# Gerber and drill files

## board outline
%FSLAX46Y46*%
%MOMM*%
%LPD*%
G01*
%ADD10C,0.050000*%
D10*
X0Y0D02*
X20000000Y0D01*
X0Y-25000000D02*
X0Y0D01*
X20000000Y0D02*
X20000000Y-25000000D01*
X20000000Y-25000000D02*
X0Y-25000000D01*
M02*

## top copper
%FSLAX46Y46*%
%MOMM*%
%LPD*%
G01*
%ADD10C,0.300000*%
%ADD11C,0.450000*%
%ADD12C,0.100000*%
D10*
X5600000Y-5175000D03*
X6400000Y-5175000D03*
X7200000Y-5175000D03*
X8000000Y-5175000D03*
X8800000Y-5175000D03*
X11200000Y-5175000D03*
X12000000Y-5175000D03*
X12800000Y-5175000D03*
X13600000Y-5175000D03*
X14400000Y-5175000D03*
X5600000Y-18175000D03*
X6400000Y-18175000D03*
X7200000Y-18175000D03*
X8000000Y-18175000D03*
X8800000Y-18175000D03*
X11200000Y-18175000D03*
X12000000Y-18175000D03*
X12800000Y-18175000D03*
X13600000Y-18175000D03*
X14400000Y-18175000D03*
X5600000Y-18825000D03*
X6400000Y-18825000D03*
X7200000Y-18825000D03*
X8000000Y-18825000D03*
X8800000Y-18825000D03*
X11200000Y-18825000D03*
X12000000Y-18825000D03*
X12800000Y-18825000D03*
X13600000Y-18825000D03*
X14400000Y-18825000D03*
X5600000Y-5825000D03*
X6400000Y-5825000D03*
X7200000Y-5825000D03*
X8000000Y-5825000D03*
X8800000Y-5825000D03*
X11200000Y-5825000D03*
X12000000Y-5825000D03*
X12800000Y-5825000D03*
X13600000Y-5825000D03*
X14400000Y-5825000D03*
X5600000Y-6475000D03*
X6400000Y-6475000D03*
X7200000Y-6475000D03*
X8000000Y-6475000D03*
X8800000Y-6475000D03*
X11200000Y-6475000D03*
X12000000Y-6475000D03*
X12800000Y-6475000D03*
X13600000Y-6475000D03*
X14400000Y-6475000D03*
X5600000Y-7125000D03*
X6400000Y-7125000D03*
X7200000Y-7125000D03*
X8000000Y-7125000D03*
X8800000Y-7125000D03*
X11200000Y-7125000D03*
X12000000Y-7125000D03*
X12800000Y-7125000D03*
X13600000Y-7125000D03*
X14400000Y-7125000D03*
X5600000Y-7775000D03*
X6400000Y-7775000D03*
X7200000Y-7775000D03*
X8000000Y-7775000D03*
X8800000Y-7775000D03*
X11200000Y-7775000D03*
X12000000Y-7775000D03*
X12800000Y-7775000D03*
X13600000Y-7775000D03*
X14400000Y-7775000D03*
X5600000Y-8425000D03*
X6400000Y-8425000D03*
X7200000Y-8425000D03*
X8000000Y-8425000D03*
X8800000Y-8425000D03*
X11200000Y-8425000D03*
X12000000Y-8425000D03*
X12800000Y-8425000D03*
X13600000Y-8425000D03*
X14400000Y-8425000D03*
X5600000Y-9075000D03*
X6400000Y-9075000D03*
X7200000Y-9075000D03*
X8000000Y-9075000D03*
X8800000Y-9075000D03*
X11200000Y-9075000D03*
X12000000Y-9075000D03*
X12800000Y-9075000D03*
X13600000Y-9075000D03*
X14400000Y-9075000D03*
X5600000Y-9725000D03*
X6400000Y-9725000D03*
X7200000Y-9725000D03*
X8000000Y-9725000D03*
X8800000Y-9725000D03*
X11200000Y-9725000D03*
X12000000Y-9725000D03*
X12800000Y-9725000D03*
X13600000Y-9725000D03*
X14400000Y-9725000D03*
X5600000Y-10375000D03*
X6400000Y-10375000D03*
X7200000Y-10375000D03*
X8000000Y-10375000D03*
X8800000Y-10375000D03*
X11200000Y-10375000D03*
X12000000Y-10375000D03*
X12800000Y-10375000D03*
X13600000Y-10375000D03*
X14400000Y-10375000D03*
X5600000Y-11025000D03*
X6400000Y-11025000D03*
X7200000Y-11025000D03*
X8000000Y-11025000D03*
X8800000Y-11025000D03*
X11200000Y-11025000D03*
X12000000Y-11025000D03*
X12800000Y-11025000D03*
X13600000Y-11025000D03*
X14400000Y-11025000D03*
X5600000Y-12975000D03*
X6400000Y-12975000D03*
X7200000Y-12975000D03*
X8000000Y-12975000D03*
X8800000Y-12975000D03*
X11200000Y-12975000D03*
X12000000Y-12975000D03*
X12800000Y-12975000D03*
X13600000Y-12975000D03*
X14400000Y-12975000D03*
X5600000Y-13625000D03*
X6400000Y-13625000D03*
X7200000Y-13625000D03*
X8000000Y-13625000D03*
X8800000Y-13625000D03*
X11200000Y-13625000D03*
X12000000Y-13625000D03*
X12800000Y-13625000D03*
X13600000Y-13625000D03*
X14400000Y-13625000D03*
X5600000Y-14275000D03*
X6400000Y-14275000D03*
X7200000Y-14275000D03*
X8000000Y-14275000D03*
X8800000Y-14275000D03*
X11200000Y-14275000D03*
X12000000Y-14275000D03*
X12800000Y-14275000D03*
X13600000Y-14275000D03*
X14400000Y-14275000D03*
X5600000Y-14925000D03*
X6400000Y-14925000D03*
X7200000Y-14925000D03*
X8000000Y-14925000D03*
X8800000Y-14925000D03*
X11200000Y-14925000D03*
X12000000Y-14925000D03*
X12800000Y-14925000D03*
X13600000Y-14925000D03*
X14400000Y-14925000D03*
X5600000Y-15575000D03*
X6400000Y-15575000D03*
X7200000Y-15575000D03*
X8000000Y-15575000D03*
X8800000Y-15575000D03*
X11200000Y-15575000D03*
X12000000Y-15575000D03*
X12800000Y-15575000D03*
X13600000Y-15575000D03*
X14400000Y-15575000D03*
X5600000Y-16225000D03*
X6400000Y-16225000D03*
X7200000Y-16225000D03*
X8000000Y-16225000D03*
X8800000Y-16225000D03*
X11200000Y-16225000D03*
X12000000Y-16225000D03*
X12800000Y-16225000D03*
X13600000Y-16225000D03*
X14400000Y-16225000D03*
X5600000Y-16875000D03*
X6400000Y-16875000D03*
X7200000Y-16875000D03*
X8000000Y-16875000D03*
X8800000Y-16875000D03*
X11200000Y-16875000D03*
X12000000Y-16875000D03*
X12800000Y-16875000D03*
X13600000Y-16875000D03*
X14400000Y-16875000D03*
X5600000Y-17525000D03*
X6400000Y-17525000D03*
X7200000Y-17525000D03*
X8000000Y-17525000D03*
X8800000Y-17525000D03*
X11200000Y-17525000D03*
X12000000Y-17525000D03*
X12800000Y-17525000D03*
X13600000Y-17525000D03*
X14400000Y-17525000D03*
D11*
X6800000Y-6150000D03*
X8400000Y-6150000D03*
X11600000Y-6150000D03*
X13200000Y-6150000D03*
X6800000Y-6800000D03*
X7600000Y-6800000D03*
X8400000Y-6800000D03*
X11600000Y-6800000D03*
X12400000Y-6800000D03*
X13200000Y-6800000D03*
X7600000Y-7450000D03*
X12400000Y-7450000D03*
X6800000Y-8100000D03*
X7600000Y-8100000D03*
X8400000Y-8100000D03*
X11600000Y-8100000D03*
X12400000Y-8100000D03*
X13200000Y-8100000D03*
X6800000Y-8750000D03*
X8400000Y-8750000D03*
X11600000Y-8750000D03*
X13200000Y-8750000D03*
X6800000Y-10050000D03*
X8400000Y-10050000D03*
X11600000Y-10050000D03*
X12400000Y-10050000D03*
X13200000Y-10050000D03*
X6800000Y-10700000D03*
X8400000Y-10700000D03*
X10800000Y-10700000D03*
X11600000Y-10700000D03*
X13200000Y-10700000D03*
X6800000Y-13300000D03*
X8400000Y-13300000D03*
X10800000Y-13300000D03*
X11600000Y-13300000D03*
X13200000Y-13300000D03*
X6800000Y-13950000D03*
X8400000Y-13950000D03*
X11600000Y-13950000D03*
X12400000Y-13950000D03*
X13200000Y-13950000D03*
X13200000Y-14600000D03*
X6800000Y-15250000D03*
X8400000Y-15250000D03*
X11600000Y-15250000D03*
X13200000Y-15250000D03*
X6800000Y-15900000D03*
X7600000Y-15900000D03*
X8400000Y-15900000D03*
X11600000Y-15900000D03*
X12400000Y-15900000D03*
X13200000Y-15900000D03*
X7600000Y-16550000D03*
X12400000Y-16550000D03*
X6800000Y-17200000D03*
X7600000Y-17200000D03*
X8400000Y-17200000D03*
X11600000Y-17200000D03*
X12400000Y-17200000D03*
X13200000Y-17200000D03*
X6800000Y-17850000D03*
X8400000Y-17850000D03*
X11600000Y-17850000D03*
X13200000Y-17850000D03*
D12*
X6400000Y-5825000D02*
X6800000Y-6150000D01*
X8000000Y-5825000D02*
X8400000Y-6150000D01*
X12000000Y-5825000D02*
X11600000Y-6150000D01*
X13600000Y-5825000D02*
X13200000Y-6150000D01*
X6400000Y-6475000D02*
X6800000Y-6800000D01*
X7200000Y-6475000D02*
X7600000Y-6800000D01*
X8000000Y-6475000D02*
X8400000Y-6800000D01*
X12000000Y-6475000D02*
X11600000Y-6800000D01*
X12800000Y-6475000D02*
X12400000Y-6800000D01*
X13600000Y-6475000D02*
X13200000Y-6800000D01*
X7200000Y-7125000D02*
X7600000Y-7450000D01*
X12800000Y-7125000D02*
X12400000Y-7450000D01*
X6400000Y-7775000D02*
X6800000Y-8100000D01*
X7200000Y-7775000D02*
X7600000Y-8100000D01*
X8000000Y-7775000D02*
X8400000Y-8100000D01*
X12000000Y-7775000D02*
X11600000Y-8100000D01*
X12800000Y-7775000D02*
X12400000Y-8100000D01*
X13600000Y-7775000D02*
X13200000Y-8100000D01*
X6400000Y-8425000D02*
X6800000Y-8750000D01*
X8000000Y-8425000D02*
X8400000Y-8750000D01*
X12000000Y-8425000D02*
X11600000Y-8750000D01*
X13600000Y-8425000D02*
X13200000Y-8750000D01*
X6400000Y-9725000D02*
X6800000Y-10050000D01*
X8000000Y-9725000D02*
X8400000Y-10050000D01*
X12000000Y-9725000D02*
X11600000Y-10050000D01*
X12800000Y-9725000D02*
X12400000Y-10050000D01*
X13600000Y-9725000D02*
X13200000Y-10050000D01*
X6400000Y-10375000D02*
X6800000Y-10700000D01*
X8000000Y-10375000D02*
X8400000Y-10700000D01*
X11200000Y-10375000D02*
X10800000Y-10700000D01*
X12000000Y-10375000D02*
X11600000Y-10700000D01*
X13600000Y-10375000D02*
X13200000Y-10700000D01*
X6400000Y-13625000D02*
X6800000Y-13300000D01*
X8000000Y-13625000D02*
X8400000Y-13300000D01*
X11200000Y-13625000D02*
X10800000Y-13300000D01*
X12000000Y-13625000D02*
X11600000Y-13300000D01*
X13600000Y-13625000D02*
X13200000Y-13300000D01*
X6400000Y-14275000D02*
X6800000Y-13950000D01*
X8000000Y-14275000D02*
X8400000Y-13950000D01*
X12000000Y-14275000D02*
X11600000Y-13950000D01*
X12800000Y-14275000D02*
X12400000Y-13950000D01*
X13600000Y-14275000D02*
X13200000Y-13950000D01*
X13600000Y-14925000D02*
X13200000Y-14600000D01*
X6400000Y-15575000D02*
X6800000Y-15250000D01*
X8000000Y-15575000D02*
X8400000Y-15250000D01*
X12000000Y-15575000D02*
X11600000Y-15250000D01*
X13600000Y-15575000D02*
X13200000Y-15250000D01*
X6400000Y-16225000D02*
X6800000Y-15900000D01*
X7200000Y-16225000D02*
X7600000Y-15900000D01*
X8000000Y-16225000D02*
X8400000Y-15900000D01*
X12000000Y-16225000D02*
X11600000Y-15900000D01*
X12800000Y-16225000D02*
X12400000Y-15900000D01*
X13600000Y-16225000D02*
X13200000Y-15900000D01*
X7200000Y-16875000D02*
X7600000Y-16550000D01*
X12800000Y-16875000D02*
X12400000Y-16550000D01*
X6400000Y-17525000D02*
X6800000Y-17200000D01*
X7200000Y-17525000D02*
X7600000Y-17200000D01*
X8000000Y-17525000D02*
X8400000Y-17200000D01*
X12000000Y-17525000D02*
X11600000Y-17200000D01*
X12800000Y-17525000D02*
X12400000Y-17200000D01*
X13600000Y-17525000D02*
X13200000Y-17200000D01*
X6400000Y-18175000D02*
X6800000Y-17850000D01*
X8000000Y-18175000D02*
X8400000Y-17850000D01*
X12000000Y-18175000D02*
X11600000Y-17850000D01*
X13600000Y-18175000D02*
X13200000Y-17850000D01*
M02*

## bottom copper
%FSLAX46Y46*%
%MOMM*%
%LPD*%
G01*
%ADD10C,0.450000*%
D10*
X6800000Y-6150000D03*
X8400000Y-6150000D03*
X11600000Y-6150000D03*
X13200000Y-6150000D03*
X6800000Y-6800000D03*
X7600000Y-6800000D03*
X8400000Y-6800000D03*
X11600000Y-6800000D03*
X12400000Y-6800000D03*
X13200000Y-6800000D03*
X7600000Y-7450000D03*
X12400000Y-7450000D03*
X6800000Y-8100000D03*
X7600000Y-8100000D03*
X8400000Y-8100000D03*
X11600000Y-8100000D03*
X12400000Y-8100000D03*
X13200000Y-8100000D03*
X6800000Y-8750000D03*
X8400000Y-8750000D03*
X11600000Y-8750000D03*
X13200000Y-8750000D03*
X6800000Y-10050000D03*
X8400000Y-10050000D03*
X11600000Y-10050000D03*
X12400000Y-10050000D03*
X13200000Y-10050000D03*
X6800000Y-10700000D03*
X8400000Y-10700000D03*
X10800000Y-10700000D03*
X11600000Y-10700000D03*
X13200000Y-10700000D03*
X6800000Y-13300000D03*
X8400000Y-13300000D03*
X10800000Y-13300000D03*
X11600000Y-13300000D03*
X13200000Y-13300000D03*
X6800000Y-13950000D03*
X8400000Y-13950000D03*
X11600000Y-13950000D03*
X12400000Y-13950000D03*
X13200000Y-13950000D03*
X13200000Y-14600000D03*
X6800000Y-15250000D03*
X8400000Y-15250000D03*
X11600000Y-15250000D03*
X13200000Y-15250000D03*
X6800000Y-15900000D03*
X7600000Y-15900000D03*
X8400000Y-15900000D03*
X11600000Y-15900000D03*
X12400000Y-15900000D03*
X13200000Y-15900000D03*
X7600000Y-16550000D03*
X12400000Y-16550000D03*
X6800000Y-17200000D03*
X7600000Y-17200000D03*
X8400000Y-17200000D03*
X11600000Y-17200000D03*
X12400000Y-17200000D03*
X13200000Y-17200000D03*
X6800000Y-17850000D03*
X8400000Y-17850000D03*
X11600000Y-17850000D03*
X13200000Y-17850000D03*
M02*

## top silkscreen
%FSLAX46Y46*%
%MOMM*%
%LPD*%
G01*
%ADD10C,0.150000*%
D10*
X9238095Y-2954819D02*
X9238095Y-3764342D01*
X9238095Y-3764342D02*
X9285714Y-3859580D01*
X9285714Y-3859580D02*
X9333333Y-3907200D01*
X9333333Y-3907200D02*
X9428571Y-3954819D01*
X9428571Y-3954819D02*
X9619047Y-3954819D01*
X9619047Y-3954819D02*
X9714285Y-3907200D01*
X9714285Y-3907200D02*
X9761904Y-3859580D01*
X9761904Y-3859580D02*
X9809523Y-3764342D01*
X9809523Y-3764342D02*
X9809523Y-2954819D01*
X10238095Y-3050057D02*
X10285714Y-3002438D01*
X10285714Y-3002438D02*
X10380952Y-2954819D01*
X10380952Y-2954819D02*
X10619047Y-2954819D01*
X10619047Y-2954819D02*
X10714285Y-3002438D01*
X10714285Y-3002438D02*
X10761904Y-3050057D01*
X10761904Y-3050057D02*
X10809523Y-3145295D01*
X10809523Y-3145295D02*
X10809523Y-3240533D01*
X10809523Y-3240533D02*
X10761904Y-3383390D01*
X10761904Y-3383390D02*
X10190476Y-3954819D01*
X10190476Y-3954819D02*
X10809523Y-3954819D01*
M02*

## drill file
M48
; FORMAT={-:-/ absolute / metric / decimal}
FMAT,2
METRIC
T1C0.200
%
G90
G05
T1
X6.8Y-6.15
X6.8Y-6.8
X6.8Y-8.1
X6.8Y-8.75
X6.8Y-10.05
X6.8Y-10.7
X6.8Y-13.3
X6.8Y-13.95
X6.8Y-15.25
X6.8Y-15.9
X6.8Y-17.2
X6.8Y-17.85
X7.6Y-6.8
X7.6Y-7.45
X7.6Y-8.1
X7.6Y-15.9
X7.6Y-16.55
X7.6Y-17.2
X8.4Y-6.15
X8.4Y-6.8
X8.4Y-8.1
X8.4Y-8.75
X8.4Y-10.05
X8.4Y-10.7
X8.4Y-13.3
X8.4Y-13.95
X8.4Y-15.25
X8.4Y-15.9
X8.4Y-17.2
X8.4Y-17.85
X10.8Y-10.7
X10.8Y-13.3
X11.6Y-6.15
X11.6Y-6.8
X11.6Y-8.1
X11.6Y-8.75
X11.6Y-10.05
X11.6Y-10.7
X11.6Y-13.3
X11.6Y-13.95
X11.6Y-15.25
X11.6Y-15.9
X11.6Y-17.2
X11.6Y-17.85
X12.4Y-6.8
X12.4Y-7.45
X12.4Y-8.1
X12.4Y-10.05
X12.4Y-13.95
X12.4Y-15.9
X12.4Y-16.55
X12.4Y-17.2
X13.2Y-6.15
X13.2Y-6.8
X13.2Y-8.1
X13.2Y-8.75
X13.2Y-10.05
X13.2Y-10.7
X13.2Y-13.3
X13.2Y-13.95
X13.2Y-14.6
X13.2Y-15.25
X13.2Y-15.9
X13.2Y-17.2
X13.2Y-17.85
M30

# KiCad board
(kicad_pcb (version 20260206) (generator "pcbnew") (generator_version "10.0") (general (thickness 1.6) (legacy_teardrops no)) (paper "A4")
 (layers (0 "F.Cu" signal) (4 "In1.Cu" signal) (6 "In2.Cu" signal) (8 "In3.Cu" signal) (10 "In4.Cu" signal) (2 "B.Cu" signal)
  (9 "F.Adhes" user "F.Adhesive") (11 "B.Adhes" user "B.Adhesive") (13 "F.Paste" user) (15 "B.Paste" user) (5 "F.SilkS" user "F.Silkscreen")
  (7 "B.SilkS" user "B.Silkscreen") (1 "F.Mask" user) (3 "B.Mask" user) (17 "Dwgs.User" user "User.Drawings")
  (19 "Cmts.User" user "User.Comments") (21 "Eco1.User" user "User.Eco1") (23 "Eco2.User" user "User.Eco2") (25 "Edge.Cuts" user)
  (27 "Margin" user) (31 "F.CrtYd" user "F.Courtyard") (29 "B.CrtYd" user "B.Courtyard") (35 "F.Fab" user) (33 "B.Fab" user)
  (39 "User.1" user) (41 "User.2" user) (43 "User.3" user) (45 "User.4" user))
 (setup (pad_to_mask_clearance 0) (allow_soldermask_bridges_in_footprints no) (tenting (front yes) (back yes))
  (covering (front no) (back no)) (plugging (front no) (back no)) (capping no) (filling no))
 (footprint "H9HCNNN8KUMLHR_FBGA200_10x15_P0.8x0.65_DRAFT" (layer "F.Cu") (at 10 12)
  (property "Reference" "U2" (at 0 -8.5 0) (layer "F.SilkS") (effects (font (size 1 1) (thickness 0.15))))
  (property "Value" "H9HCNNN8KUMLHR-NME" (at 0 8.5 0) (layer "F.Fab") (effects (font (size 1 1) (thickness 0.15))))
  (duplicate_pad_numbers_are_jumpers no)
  (pad "A1" smd circle (at -4.4 -6.825) (size 0.3 0.3) (layers "F.Cu" "F.Mask" "F.Paste"))
  (pad "A2" smd circle (at -3.6 -6.825) (size 0.3 0.3) (layers "F.Cu" "F.Mask" "F.Paste"))
  (pad "A3" smd circle (at -2.8 -6.825) (size 0.3 0.3) (layers "F.Cu" "F.Mask" "F.Paste") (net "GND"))
  (pad "A4" smd circle (at -2 -6.825) (size 0.3 0.3) (layers "F.Cu" "F.Mask" "F.Paste") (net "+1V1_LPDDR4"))
  (pad "A5" smd circle (at -1.2 -6.825) (size 0.3 0.3) (layers "F.Cu" "F.Mask" "F.Paste") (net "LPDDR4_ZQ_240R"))
  (pad "A8" smd circle (at 1.2 -6.825) (size 0.3 0.3) (layers "F.Cu" "F.Mask" "F.Paste"))
  (pad "A9" smd circle (at 2 -6.825) (size 0.3 0.3) (layers "F.Cu" "F.Mask" "F.Paste") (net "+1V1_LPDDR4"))
  (pad "A10" smd circle (at 2.8 -6.825) (size 0.3 0.3) (layers "F.Cu" "F.Mask" "F.Paste") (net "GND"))
  (pad "A11" smd circle (at 3.6 -6.825) (size 0.3 0.3) (layers "F.Cu" "F.Mask" "F.Paste"))
  (pad "A12" smd circle (at 4.4 -6.825) (size 0.3 0.3) (layers "F.Cu" "F.Mask" "F.Paste"))
  (pad "AA1" smd circle (at -4.4 6.175) (size 0.3 0.3) (layers "F.Cu" "F.Mask" "F.Paste"))
  (pad "AA2" smd circle (at -3.6 6.175) (size 0.3 0.3) (layers "F.Cu" "F.Mask" "F.Paste") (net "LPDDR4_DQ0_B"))
  (pad "AA3" smd circle (at -2.8 6.175) (size 0.3 0.3) (layers "F.Cu" "F.Mask" "F.Paste") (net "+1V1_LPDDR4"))
  (pad "AA4" smd circle (at -2 6.175) (size 0.3 0.3) (layers "F.Cu" "F.Mask" "F.Paste") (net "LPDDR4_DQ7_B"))
  (pad "AA5" smd circle (at -1.2 6.175) (size 0.3 0.3) (layers "F.Cu" "F.Mask" "F.Paste") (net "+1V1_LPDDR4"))
  (pad "AA8" smd circle (at 1.2 6.175) (size 0.3 0.3) (layers "F.Cu" "F.Mask" "F.Paste") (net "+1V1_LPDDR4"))
  (pad "AA9" smd circle (at 2 6.175) (size 0.3 0.3) (layers "F.Cu" "F.Mask" "F.Paste") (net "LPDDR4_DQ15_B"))
  (pad "AA10" smd circle (at 2.8 6.175) (size 0.3 0.3) (layers "F.Cu" "F.Mask" "F.Paste") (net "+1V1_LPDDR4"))
  (pad "AA11" smd circle (at 3.6 6.175) (size 0.3 0.3) (layers "F.Cu" "F.Mask" "F.Paste") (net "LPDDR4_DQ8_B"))
  (pad "AA12" smd circle (at 4.4 6.175) (size 0.3 0.3) (layers "F.Cu" "F.Mask" "F.Paste"))
  (pad "AB1" smd circle (at -4.4 6.825) (size 0.3 0.3) (layers "F.Cu" "F.Mask" "F.Paste"))
  (pad "AB2" smd circle (at -3.6 6.825) (size 0.3 0.3) (layers "F.Cu" "F.Mask" "F.Paste"))
  (pad "AB3" smd circle (at -2.8 6.825) (size 0.3 0.3) (layers "F.Cu" "F.Mask" "F.Paste") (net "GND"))
  (pad "AB4" smd circle (at -2 6.825) (size 0.3 0.3) (layers "F.Cu" "F.Mask" "F.Paste") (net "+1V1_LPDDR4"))
  (pad "AB5" smd circle (at -1.2 6.825) (size 0.3 0.3) (layers "F.Cu" "F.Mask" "F.Paste") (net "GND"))
  (pad "AB8" smd circle (at 1.2 6.825) (size 0.3 0.3) (layers "F.Cu" "F.Mask" "F.Paste") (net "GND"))
  (pad "AB9" smd circle (at 2 6.825) (size 0.3 0.3) (layers "F.Cu" "F.Mask" "F.Paste") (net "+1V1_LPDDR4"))
  (pad "AB10" smd circle (at 2.8 6.825) (size 0.3 0.3) (layers "F.Cu" "F.Mask" "F.Paste") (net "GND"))
  (pad "AB11" smd circle (at 3.6 6.825) (size 0.3 0.3) (layers "F.Cu" "F.Mask" "F.Paste"))
  (pad "AB12" smd circle (at 4.4 6.825) (size 0.3 0.3) (layers "F.Cu" "F.Mask" "F.Paste"))
  (pad "B1" smd circle (at -4.4 -6.175) (size 0.3 0.3) (layers "F.Cu" "F.Mask" "F.Paste"))
  (pad "B2" smd circle (at -3.6 -6.175) (size 0.3 0.3) (layers "F.Cu" "F.Mask" "F.Paste") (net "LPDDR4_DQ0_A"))
  (pad "B3" smd circle (at -2.8 -6.175) (size 0.3 0.3) (layers "F.Cu" "F.Mask" "F.Paste") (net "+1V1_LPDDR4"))
  (pad "B4" smd circle (at -2 -6.175) (size 0.3 0.3) (layers "F.Cu" "F.Mask" "F.Paste") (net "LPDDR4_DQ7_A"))
  (pad "B5" smd circle (at -1.2 -6.175) (size 0.3 0.3) (layers "F.Cu" "F.Mask" "F.Paste") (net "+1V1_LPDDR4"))
  (pad "B8" smd circle (at 1.2 -6.175) (size 0.3 0.3) (layers "F.Cu" "F.Mask" "F.Paste") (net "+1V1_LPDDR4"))
  (pad "B9" smd circle (at 2 -6.175) (size 0.3 0.3) (layers "F.Cu" "F.Mask" "F.Paste") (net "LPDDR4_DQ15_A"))
  (pad "B10" smd circle (at 2.8 -6.175) (size 0.3 0.3) (layers "F.Cu" "F.Mask" "F.Paste") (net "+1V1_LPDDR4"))
  (pad "B11" smd circle (at 3.6 -6.175) (size 0.3 0.3) (layers "F.Cu" "F.Mask" "F.Paste") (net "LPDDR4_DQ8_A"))
  (pad "B12" smd circle (at 4.4 -6.175) (size 0.3 0.3) (layers "F.Cu" "F.Mask" "F.Paste"))
  (pad "C1" smd circle (at -4.4 -5.525) (size 0.3 0.3) (layers "F.Cu" "F.Mask" "F.Paste") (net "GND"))
  (pad "C2" smd circle (at -3.6 -5.525) (size 0.3 0.3) (layers "F.Cu" "F.Mask" "F.Paste") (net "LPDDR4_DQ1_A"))
  (pad "C3" smd circle (at -2.8 -5.525) (size 0.3 0.3) (layers "F.Cu" "F.Mask" "F.Paste") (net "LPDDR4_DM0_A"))
  (pad "C4" smd circle (at -2 -5.525) (size 0.3 0.3) (layers "F.Cu" "F.Mask" "F.Paste") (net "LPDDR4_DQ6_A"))
  (pad "C5" smd circle (at -1.2 -5.525) (size 0.3 0.3) (layers "F.Cu" "F.Mask" "F.Paste") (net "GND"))
  (pad "C8" smd circle (at 1.2 -5.525) (size 0.3 0.3) (layers "F.Cu" "F.Mask" "F.Paste") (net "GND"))
  (pad "C9" smd circle (at 2 -5.525) (size 0.3 0.3) (layers "F.Cu" "F.Mask" "F.Paste") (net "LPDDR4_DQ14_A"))
  (pad "C10" smd circle (at 2.8 -5.525) (size 0.3 0.3) (layers "F.Cu" "F.Mask" "F.Paste") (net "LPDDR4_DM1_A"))
  (pad "C11" smd circle (at 3.6 -5.525) (size 0.3 0.3) (layers "F.Cu" "F.Mask" "F.Paste") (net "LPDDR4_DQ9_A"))
  (pad "C12" smd circle (at 4.4 -5.525) (size 0.3 0.3) (layers "F.Cu" "F.Mask" "F.Paste") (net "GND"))
  (pad "D1" smd circle (at -4.4 -4.875) (size 0.3 0.3) (layers "F.Cu" "F.Mask" "F.Paste") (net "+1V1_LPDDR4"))
  (pad "D2" smd circle (at -3.6 -4.875) (size 0.3 0.3) (layers "F.Cu" "F.Mask" "F.Paste") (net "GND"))
  (pad "D3" smd circle (at -2.8 -4.875) (size 0.3 0.3) (layers "F.Cu" "F.Mask" "F.Paste") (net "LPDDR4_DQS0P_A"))
  (pad "D4" smd circle (at -2 -4.875) (size 0.3 0.3) (layers "F.Cu" "F.Mask" "F.Paste") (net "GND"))
  (pad "D5" smd circle (at -1.2 -4.875) (size 0.3 0.3) (layers "F.Cu" "F.Mask" "F.Paste") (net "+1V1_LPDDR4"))
  (pad "D8" smd circle (at 1.2 -4.875) (size 0.3 0.3) (layers "F.Cu" "F.Mask" "F.Paste") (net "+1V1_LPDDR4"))
  (pad "D9" smd circle (at 2 -4.875) (size 0.3 0.3) (layers "F.Cu" "F.Mask" "F.Paste") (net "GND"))
  (pad "D10" smd circle (at 2.8 -4.875) (size 0.3 0.3) (layers "F.Cu" "F.Mask" "F.Paste") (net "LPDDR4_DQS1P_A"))
  (pad "D11" smd circle (at 3.6 -4.875) (size 0.3 0.3) (layers "F.Cu" "F.Mask" "F.Paste") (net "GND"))
  (pad "D12" smd circle (at 4.4 -4.875) (size 0.3 0.3) (layers "F.Cu" "F.Mask" "F.Paste") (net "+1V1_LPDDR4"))
  (pad "E1" smd circle (at -4.4 -4.225) (size 0.3 0.3) (layers "F.Cu" "F.Mask" "F.Paste") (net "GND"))
  (pad "E2" smd circle (at -3.6 -4.225) (size 0.3 0.3) (layers "F.Cu" "F.Mask" "F.Paste") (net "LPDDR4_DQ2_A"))
  (pad "E3" smd circle (at -2.8 -4.225) (size 0.3 0.3) (layers "F.Cu" "F.Mask" "F.Paste") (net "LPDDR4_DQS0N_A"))
  (pad "E4" smd circle (at -2 -4.225) (size 0.3 0.3) (layers "F.Cu" "F.Mask" "F.Paste") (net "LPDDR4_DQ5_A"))
  (pad "E5" smd circle (at -1.2 -4.225) (size 0.3 0.3) (layers "F.Cu" "F.Mask" "F.Paste") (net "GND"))
  (pad "E8" smd circle (at 1.2 -4.225) (size 0.3 0.3) (layers "F.Cu" "F.Mask" "F.Paste") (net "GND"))
  (pad "E9" smd circle (at 2 -4.225) (size 0.3 0.3) (layers "F.Cu" "F.Mask" "F.Paste") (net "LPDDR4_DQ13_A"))
  (pad "E10" smd circle (at 2.8 -4.225) (size 0.3 0.3) (layers "F.Cu" "F.Mask" "F.Paste") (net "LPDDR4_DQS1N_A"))
  (pad "E11" smd circle (at 3.6 -4.225) (size 0.3 0.3) (layers "F.Cu" "F.Mask" "F.Paste") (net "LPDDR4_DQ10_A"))
  (pad "E12" smd circle (at 4.4 -4.225) (size 0.3 0.3) (layers "F.Cu" "F.Mask" "F.Paste") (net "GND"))
  (pad "F1" smd circle (at -4.4 -3.575) (size 0.3 0.3) (layers "F.Cu" "F.Mask" "F.Paste") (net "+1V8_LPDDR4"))
  (pad "F2" smd circle (at -3.6 -3.575) (size 0.3 0.3) (layers "F.Cu" "F.Mask" "F.Paste") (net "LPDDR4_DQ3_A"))
  (pad "F3" smd circle (at -2.8 -3.575) (size 0.3 0.3) (layers "F.Cu" "F.Mask" "F.Paste") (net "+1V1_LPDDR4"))
  (pad "F4" smd circle (at -2 -3.575) (size 0.3 0.3) (layers "F.Cu" "F.Mask" "F.Paste") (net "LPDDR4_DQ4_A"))
  (pad "F5" smd circle (at -1.2 -3.575) (size 0.3 0.3) (layers "F.Cu" "F.Mask" "F.Paste") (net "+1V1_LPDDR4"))
  (pad "F8" smd circle (at 1.2 -3.575) (size 0.3 0.3) (layers "F.Cu" "F.Mask" "F.Paste") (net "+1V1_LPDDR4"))
  (pad "F9" smd circle (at 2 -3.575) (size 0.3 0.3) (layers "F.Cu" "F.Mask" "F.Paste") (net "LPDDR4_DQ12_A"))
  (pad "F10" smd circle (at 2.8 -3.575) (size 0.3 0.3) (layers "F.Cu" "F.Mask" "F.Paste") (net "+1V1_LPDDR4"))
  (pad "F11" smd circle (at 3.6 -3.575) (size 0.3 0.3) (layers "F.Cu" "F.Mask" "F.Paste") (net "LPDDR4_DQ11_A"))
  (pad "F12" smd circle (at 4.4 -3.575) (size 0.3 0.3) (layers "F.Cu" "F.Mask" "F.Paste") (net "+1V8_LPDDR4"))
  (pad "G1" smd circle (at -4.4 -2.925) (size 0.3 0.3) (layers "F.Cu" "F.Mask" "F.Paste") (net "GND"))
  (pad "G2" smd circle (at -3.6 -2.925) (size 0.3 0.3) (layers "F.Cu" "F.Mask" "F.Paste") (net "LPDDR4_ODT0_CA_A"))
  (pad "G3" smd circle (at -2.8 -2.925) (size 0.3 0.3) (layers "F.Cu" "F.Mask" "F.Paste") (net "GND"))
  (pad "G4" smd circle (at -2 -2.925) (size 0.3 0.3) (layers "F.Cu" "F.Mask" "F.Paste") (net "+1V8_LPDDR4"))
  (pad "G5" smd circle (at -1.2 -2.925) (size 0.3 0.3) (layers "F.Cu" "F.Mask" "F.Paste") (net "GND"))
  (pad "G8" smd circle (at 1.2 -2.925) (size 0.3 0.3) (layers "F.Cu" "F.Mask" "F.Paste") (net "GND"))
  (pad "G9" smd circle (at 2 -2.925) (size 0.3 0.3) (layers "F.Cu" "F.Mask" "F.Paste") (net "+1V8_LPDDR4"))
  (pad "G10" smd circle (at 2.8 -2.925) (size 0.3 0.3) (layers "F.Cu" "F.Mask" "F.Paste") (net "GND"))
  (pad "G11" smd circle (at 3.6 -2.925) (size 0.3 0.3) (layers "F.Cu" "F.Mask" "F.Paste"))
  (pad "G12" smd circle (at 4.4 -2.925) (size 0.3 0.3) (layers "F.Cu" "F.Mask" "F.Paste") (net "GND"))
  (pad "H1" smd circle (at -4.4 -2.275) (size 0.3 0.3) (layers "F.Cu" "F.Mask" "F.Paste") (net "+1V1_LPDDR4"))
  (pad "H2" smd circle (at -3.6 -2.275) (size 0.3 0.3) (layers "F.Cu" "F.Mask" "F.Paste") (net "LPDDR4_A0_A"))
  (pad "H3" smd circle (at -2.8 -2.275) (size 0.3 0.3) (layers "F.Cu" "F.Mask" "F.Paste"))
  (pad "H4" smd circle (at -2 -2.275) (size 0.3 0.3) (layers "F.Cu" "F.Mask" "F.Paste") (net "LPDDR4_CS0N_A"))
  (pad "H5" smd circle (at -1.2 -2.275) (size 0.3 0.3) (layers "F.Cu" "F.Mask" "F.Paste") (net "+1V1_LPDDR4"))
  (pad "H8" smd circle (at 1.2 -2.275) (size 0.3 0.3) (layers "F.Cu" "F.Mask" "F.Paste") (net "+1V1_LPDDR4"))
  (pad "H9" smd circle (at 2 -2.275) (size 0.3 0.3) (layers "F.Cu" "F.Mask" "F.Paste") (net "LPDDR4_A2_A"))
  (pad "H10" smd circle (at 2.8 -2.275) (size 0.3 0.3) (layers "F.Cu" "F.Mask" "F.Paste") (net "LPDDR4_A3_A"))
  (pad "H11" smd circle (at 3.6 -2.275) (size 0.3 0.3) (layers "F.Cu" "F.Mask" "F.Paste") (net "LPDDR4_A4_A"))
  (pad "H12" smd circle (at 4.4 -2.275) (size 0.3 0.3) (layers "F.Cu" "F.Mask" "F.Paste") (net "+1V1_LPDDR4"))
  (pad "J1" smd circle (at -4.4 -1.625) (size 0.3 0.3) (layers "F.Cu" "F.Mask" "F.Paste") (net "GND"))
  (pad "J2" smd circle (at -3.6 -1.625) (size 0.3 0.3) (layers "F.Cu" "F.Mask" "F.Paste") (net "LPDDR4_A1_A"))
  (pad "J3" smd circle (at -2.8 -1.625) (size 0.3 0.3) (layers "F.Cu" "F.Mask" "F.Paste") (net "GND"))
  (pad "J4" smd circle (at -2 -1.625) (size 0.3 0.3) (layers "F.Cu" "F.Mask" "F.Paste") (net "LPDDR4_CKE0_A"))
  (pad "J5" smd circle (at -1.2 -1.625) (size 0.3 0.3) (layers "F.Cu" "F.Mask" "F.Paste"))
  (pad "J8" smd circle (at 1.2 -1.625) (size 0.3 0.3) (layers "F.Cu" "F.Mask" "F.Paste") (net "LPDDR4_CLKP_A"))
  (pad "J9" smd circle (at 2 -1.625) (size 0.3 0.3) (layers "F.Cu" "F.Mask" "F.Paste") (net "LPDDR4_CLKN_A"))
  (pad "J10" smd circle (at 2.8 -1.625) (size 0.3 0.3) (layers "F.Cu" "F.Mask" "F.Paste") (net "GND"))
  (pad "J11" smd circle (at 3.6 -1.625) (size 0.3 0.3) (layers "F.Cu" "F.Mask" "F.Paste") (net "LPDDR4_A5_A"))
  (pad "J12" smd circle (at 4.4 -1.625) (size 0.3 0.3) (layers "F.Cu" "F.Mask" "F.Paste") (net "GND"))
  (pad "K1" smd circle (at -4.4 -0.975) (size 0.3 0.3) (layers "F.Cu" "F.Mask" "F.Paste") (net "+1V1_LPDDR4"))
  (pad "K2" smd circle (at -3.6 -0.975) (size 0.3 0.3) (layers "F.Cu" "F.Mask" "F.Paste") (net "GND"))
  (pad "K3" smd circle (at -2.8 -0.975) (size 0.3 0.3) (layers "F.Cu" "F.Mask" "F.Paste") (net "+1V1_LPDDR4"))
  (pad "K4" smd circle (at -2 -0.975) (size 0.3 0.3) (layers "F.Cu" "F.Mask" "F.Paste") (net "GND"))
  (pad "K5" smd circle (at -1.2 -0.975) (size 0.3 0.3) (layers "F.Cu" "F.Mask" "F.Paste"))
  (pad "K8" smd circle (at 1.2 -0.975) (size 0.3 0.3) (layers "F.Cu" "F.Mask" "F.Paste"))
  (pad "K9" smd circle (at 2 -0.975) (size 0.3 0.3) (layers "F.Cu" "F.Mask" "F.Paste") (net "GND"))
  (pad "K10" smd circle (at 2.8 -0.975) (size 0.3 0.3) (layers "F.Cu" "F.Mask" "F.Paste") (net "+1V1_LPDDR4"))
  (pad "K11" smd circle (at 3.6 -0.975) (size 0.3 0.3) (layers "F.Cu" "F.Mask" "F.Paste") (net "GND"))
  (pad "K12" smd circle (at 4.4 -0.975) (size 0.3 0.3) (layers "F.Cu" "F.Mask" "F.Paste") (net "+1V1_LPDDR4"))
  (pad "N1" smd circle (at -4.4 0.975) (size 0.3 0.3) (layers "F.Cu" "F.Mask" "F.Paste") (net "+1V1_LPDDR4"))
  (pad "N2" smd circle (at -3.6 0.975) (size 0.3 0.3) (layers "F.Cu" "F.Mask" "F.Paste") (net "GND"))
  (pad "N3" smd circle (at -2.8 0.975) (size 0.3 0.3) (layers "F.Cu" "F.Mask" "F.Paste") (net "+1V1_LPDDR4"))
  (pad "N4" smd circle (at -2 0.975) (size 0.3 0.3) (layers "F.Cu" "F.Mask" "F.Paste") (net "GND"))
  (pad "N5" smd circle (at -1.2 0.975) (size 0.3 0.3) (layers "F.Cu" "F.Mask" "F.Paste"))
  (pad "N8" smd circle (at 1.2 0.975) (size 0.3 0.3) (layers "F.Cu" "F.Mask" "F.Paste"))
  (pad "N9" smd circle (at 2 0.975) (size 0.3 0.3) (layers "F.Cu" "F.Mask" "F.Paste") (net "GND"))
  (pad "N10" smd circle (at 2.8 0.975) (size 0.3 0.3) (layers "F.Cu" "F.Mask" "F.Paste") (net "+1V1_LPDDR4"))
  (pad "N11" smd circle (at 3.6 0.975) (size 0.3 0.3) (layers "F.Cu" "F.Mask" "F.Paste") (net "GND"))
  (pad "N12" smd circle (at 4.4 0.975) (size 0.3 0.3) (layers "F.Cu" "F.Mask" "F.Paste") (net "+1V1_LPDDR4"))
  (pad "P1" smd circle (at -4.4 1.625) (size 0.3 0.3) (layers "F.Cu" "F.Mask" "F.Paste") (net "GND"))
  (pad "P2" smd circle (at -3.6 1.625) (size 0.3 0.3) (layers "F.Cu" "F.Mask" "F.Paste") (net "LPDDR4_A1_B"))
  (pad "P3" smd circle (at -2.8 1.625) (size 0.3 0.3) (layers "F.Cu" "F.Mask" "F.Paste") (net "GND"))
  (pad "P4" smd circle (at -2 1.625) (size 0.3 0.3) (layers "F.Cu" "F.Mask" "F.Paste") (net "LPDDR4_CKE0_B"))
  (pad "P5" smd circle (at -1.2 1.625) (size 0.3 0.3) (layers "F.Cu" "F.Mask" "F.Paste"))
  (pad "P8" smd circle (at 1.2 1.625) (size 0.3 0.3) (layers "F.Cu" "F.Mask" "F.Paste") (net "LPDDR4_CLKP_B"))
  (pad "P9" smd circle (at 2 1.625) (size 0.3 0.3) (layers "F.Cu" "F.Mask" "F.Paste") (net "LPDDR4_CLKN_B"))
  (pad "P10" smd circle (at 2.8 1.625) (size 0.3 0.3) (layers "F.Cu" "F.Mask" "F.Paste") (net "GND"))
  (pad "P11" smd circle (at 3.6 1.625) (size 0.3 0.3) (layers "F.Cu" "F.Mask" "F.Paste") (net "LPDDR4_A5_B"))
  (pad "P12" smd circle (at 4.4 1.625) (size 0.3 0.3) (layers "F.Cu" "F.Mask" "F.Paste") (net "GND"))
  (pad "R1" smd circle (at -4.4 2.275) (size 0.3 0.3) (layers "F.Cu" "F.Mask" "F.Paste") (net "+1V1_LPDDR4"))
  (pad "R2" smd circle (at -3.6 2.275) (size 0.3 0.3) (layers "F.Cu" "F.Mask" "F.Paste") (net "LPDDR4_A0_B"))
  (pad "R3" smd circle (at -2.8 2.275) (size 0.3 0.3) (layers "F.Cu" "F.Mask" "F.Paste"))
  (pad "R4" smd circle (at -2 2.275) (size 0.3 0.3) (layers "F.Cu" "F.Mask" "F.Paste") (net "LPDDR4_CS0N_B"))
  (pad "R5" smd circle (at -1.2 2.275) (size 0.3 0.3) (layers "F.Cu" "F.Mask" "F.Paste") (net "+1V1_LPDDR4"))
  (pad "R8" smd circle (at 1.2 2.275) (size 0.3 0.3) (layers "F.Cu" "F.Mask" "F.Paste") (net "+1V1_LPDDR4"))
  (pad "R9" smd circle (at 2 2.275) (size 0.3 0.3) (layers "F.Cu" "F.Mask" "F.Paste") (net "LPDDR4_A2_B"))
  (pad "R10" smd circle (at 2.8 2.275) (size 0.3 0.3) (layers "F.Cu" "F.Mask" "F.Paste") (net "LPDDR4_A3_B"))
  (pad "R11" smd circle (at 3.6 2.275) (size 0.3 0.3) (layers "F.Cu" "F.Mask" "F.Paste") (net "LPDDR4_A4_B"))
  (pad "R12" smd circle (at 4.4 2.275) (size 0.3 0.3) (layers "F.Cu" "F.Mask" "F.Paste") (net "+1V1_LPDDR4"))
  (pad "T1" smd circle (at -4.4 2.925) (size 0.3 0.3) (layers "F.Cu" "F.Mask" "F.Paste") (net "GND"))
  (pad "T2" smd circle (at -3.6 2.925) (size 0.3 0.3) (layers "F.Cu" "F.Mask" "F.Paste") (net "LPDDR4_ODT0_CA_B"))
  (pad "T3" smd circle (at -2.8 2.925) (size 0.3 0.3) (layers "F.Cu" "F.Mask" "F.Paste") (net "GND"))
  (pad "T4" smd circle (at -2 2.925) (size 0.3 0.3) (layers "F.Cu" "F.Mask" "F.Paste") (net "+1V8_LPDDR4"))
  (pad "T5" smd circle (at -1.2 2.925) (size 0.3 0.3) (layers "F.Cu" "F.Mask" "F.Paste") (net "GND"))
  (pad "T8" smd circle (at 1.2 2.925) (size 0.3 0.3) (layers "F.Cu" "F.Mask" "F.Paste") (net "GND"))
  (pad "T9" smd circle (at 2 2.925) (size 0.3 0.3) (layers "F.Cu" "F.Mask" "F.Paste") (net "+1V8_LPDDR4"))
  (pad "T10" smd circle (at 2.8 2.925) (size 0.3 0.3) (layers "F.Cu" "F.Mask" "F.Paste") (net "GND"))
  (pad "T11" smd circle (at 3.6 2.925) (size 0.3 0.3) (layers "F.Cu" "F.Mask" "F.Paste") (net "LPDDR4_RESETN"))
  (pad "T12" smd circle (at 4.4 2.925) (size 0.3 0.3) (layers "F.Cu" "F.Mask" "F.Paste") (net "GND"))
  (pad "U1" smd circle (at -4.4 3.575) (size 0.3 0.3) (layers "F.Cu" "F.Mask" "F.Paste") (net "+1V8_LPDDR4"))
  (pad "U2" smd circle (at -3.6 3.575) (size 0.3 0.3) (layers "F.Cu" "F.Mask" "F.Paste") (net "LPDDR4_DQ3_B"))
  (pad "U3" smd circle (at -2.8 3.575) (size 0.3 0.3) (layers "F.Cu" "F.Mask" "F.Paste") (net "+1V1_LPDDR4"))
  (pad "U4" smd circle (at -2 3.575) (size 0.3 0.3) (layers "F.Cu" "F.Mask" "F.Paste") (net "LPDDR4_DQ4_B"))
  (pad "U5" smd circle (at -1.2 3.575) (size 0.3 0.3) (layers "F.Cu" "F.Mask" "F.Paste") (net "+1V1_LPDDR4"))
  (pad "U8" smd circle (at 1.2 3.575) (size 0.3 0.3) (layers "F.Cu" "F.Mask" "F.Paste") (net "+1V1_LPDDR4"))
  (pad "U9" smd circle (at 2 3.575) (size 0.3 0.3) (layers "F.Cu" "F.Mask" "F.Paste") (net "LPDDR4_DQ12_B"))
  (pad "U10" smd circle (at 2.8 3.575) (size 0.3 0.3) (layers "F.Cu" "F.Mask" "F.Paste") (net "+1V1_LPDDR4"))
  (pad "U11" smd circle (at 3.6 3.575) (size 0.3 0.3) (layers "F.Cu" "F.Mask" "F.Paste") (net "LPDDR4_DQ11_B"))
  (pad "U12" smd circle (at 4.4 3.575) (size 0.3 0.3) (layers "F.Cu" "F.Mask" "F.Paste") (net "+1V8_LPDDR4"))
  (pad "V1" smd circle (at -4.4 4.225) (size 0.3 0.3) (layers "F.Cu" "F.Mask" "F.Paste") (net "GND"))
  (pad "V2" smd circle (at -3.6 4.225) (size 0.3 0.3) (layers "F.Cu" "F.Mask" "F.Paste") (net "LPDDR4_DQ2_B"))
  (pad "V3" smd circle (at -2.8 4.225) (size 0.3 0.3) (layers "F.Cu" "F.Mask" "F.Paste") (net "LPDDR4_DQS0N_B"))
  (pad "V4" smd circle (at -2 4.225) (size 0.3 0.3) (layers "F.Cu" "F.Mask" "F.Paste") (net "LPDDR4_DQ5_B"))
  (pad "V5" smd circle (at -1.2 4.225) (size 0.3 0.3) (layers "F.Cu" "F.Mask" "F.Paste") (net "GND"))
  (pad "V8" smd circle (at 1.2 4.225) (size 0.3 0.3) (layers "F.Cu" "F.Mask" "F.Paste") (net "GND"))
  (pad "V9" smd circle (at 2 4.225) (size 0.3 0.3) (layers "F.Cu" "F.Mask" "F.Paste") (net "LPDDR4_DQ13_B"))
  (pad "V10" smd circle (at 2.8 4.225) (size 0.3 0.3) (layers "F.Cu" "F.Mask" "F.Paste") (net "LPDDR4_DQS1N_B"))
  (pad "V11" smd circle (at 3.6 4.225) (size 0.3 0.3) (layers "F.Cu" "F.Mask" "F.Paste") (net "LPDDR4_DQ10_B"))
  (pad "V12" smd circle (at 4.4 4.225) (size 0.3 0.3) (layers "F.Cu" "F.Mask" "F.Paste") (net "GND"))
  (pad "W1" smd circle (at -4.4 4.875) (size 0.3 0.3) (layers "F.Cu" "F.Mask" "F.Paste") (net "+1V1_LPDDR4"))
  (pad "W2" smd circle (at -3.6 4.875) (size 0.3 0.3) (layers "F.Cu" "F.Mask" "F.Paste") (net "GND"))
  (pad "W3" smd circle (at -2.8 4.875) (size 0.3 0.3) (layers "F.Cu" "F.Mask" "F.Paste") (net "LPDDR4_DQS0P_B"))
  (pad "W4" smd circle (at -2 4.875) (size 0.3 0.3) (layers "F.Cu" "F.Mask" "F.Paste") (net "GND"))
  (pad "W5" smd circle (at -1.2 4.875) (size 0.3 0.3) (layers "F.Cu" "F.Mask" "F.Paste") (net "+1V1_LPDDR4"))
  (pad "W8" smd circle (at 1.2 4.875) (size 0.3 0.3) (layers "F.Cu" "F.Mask" "F.Paste") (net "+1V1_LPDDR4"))
  (pad "W9" smd circle (at 2 4.875) (size 0.3 0.3) (layers "F.Cu" "F.Mask" "F.Paste") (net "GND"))
  (pad "W10" smd circle (at 2.8 4.875) (size 0.3 0.3) (layers "F.Cu" "F.Mask" "F.Paste") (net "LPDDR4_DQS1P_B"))
  (pad "W11" smd circle (at 3.6 4.875) (size 0.3 0.3) (layers "F.Cu" "F.Mask" "F.Paste") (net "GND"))
  (pad "W12" smd circle (at 4.4 4.875) (size 0.3 0.3) (layers "F.Cu" "F.Mask" "F.Paste") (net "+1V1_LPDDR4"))
  (pad "Y1" smd circle (at -4.4 5.525) (size 0.3 0.3) (layers "F.Cu" "F.Mask" "F.Paste") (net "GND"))
  (pad "Y2" smd circle (at -3.6 5.525) (size 0.3 0.3) (layers "F.Cu" "F.Mask" "F.Paste") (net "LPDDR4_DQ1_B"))
  (pad "Y3" smd circle (at -2.8 5.525) (size 0.3 0.3) (layers "F.Cu" "F.Mask" "F.Paste") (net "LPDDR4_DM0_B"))
  (pad "Y4" smd circle (at -2 5.525) (size 0.3 0.3) (layers "F.Cu" "F.Mask" "F.Paste") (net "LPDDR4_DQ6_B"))
  (pad "Y5" smd circle (at -1.2 5.525) (size 0.3 0.3) (layers "F.Cu" "F.Mask" "F.Paste") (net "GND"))
  (pad "Y8" smd circle (at 1.2 5.525) (size 0.3 0.3) (layers "F.Cu" "F.Mask" "F.Paste") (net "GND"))
  (pad "Y9" smd circle (at 2 5.525) (size 0.3 0.3) (layers "F.Cu" "F.Mask" "F.Paste") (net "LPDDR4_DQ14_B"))
  (pad "Y10" smd circle (at 2.8 5.525) (size 0.3 0.3) (layers "F.Cu" "F.Mask" "F.Paste") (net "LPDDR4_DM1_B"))
  (pad "Y11" smd circle (at 3.6 5.525) (size 0.3 0.3) (layers "F.Cu" "F.Mask" "F.Paste") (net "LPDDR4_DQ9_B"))
  (pad "Y12" smd circle (at 4.4 5.525) (size 0.3 0.3) (layers "F.Cu" "F.Mask" "F.Paste") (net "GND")))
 (gr_line (start 0 0) (end 20 0) (stroke (width 0.05) (type default)) (layer "Edge.Cuts"))
 (gr_line (start 0 25) (end 0 0) (stroke (width 0.05) (type default)) (layer "Edge.Cuts"))
 (gr_line (start 20 0) (end 20 25) (stroke (width 0.05) (type default)) (layer "Edge.Cuts"))
 (gr_line (start 20 25) (end 0 25) (stroke (width 0.05) (type default)) (layer "Edge.Cuts"))
 (segment (start 6.4 5.825) (end 6.8 6.15) (width 0.1) (layer "F.Cu") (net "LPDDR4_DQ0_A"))
 (via (at 6.8 6.15) (size 0.45) (drill 0.2) (layers "F.Cu" "B.Cu") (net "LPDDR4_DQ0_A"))
 (segment (start 8 5.825) (end 8.4 6.15) (width 0.1) (layer "F.Cu") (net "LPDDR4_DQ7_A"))
 (via (at 8.4 6.15) (size 0.45) (drill 0.2) (layers "F.Cu" "B.Cu") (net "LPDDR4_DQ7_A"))
 (segment (start 12 5.825) (end 11.6 6.15) (width 0.1) (layer "F.Cu") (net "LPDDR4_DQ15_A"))
 (via (at 11.6 6.15) (size 0.45) (drill 0.2) (layers "F.Cu" "B.Cu") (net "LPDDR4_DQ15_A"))
 (segment (start 13.6 5.825) (end 13.2 6.15) (width 0.1) (layer "F.Cu") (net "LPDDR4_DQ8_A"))
 (via (at 13.2 6.15) (size 0.45) (drill 0.2) (layers "F.Cu" "B.Cu") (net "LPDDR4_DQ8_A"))
 (segment (start 6.4 6.475) (end 6.8 6.8) (width 0.1) (layer "F.Cu") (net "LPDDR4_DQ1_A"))
 (via (at 6.8 6.8) (size 0.45) (drill 0.2) (layers "F.Cu" "B.Cu") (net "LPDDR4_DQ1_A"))
 (segment (start 7.2 6.475) (end 7.6 6.8) (width 0.1) (layer "F.Cu") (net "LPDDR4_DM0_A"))
 (via (at 7.6 6.8) (size 0.45) (drill 0.2) (layers "F.Cu" "B.Cu") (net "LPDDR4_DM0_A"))
 (segment (start 8 6.475) (end 8.4 6.8) (width 0.1) (layer "F.Cu") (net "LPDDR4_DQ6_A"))
 (via (at 8.4 6.8) (size 0.45) (drill 0.2) (layers "F.Cu" "B.Cu") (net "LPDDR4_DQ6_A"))
 (segment (start 12 6.475) (end 11.6 6.8) (width 0.1) (layer "F.Cu") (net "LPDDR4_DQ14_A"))
 (via (at 11.6 6.8) (size 0.45) (drill 0.2) (layers "F.Cu" "B.Cu") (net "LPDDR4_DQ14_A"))
 (segment (start 12.8 6.475) (end 12.4 6.8) (width 0.1) (layer "F.Cu") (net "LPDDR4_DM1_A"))
 (via (at 12.4 6.8) (size 0.45) (drill 0.2) (layers "F.Cu" "B.Cu") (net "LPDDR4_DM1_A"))
 (segment (start 13.6 6.475) (end 13.2 6.8) (width 0.1) (layer "F.Cu") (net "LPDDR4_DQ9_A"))
 (via (at 13.2 6.8) (size 0.45) (drill 0.2) (layers "F.Cu" "B.Cu") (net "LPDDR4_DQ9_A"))
 (segment (start 7.2 7.125) (end 7.6 7.45) (width 0.1) (layer "F.Cu") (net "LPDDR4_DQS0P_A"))
 (via (at 7.6 7.45) (size 0.45) (drill 0.2) (layers "F.Cu" "B.Cu") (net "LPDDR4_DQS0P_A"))
 (segment (start 12.8 7.125) (end 12.4 7.45) (width 0.1) (layer "F.Cu") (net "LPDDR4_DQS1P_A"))
 (via (at 12.4 7.45) (size 0.45) (drill 0.2) (layers "F.Cu" "B.Cu") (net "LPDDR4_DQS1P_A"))
 (segment (start 6.4 7.775) (end 6.8 8.1) (width 0.1) (layer "F.Cu") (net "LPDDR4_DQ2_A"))
 (via (at 6.8 8.1) (size 0.45) (drill 0.2) (layers "F.Cu" "B.Cu") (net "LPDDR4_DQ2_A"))
 (segment (start 7.2 7.775) (end 7.6 8.1) (width 0.1) (layer "F.Cu") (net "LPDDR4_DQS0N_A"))
 (via (at 7.6 8.1) (size 0.45) (drill 0.2) (layers "F.Cu" "B.Cu") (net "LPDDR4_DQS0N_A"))
 (segment (start 8 7.775) (end 8.4 8.1) (width 0.1) (layer "F.Cu") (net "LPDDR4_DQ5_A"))
 (via (at 8.4 8.1) (size 0.45) (drill 0.2) (layers "F.Cu" "B.Cu") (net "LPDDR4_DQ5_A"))
 (segment (start 12 7.775) (end 11.6 8.1) (width 0.1) (layer "F.Cu") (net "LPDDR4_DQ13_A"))
 (via (at 11.6 8.1) (size 0.45) (drill 0.2) (layers "F.Cu" "B.Cu") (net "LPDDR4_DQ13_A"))
 (segment (start 12.8 7.775) (end 12.4 8.1) (width 0.1) (layer "F.Cu") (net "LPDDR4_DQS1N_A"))
 (via (at 12.4 8.1) (size 0.45) (drill 0.2) (layers "F.Cu" "B.Cu") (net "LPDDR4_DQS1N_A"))
 (segment (start 13.6 7.775) (end 13.2 8.1) (width 0.1) (layer "F.Cu") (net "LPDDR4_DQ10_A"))
 (via (at 13.2 8.1) (size 0.45) (drill 0.2) (layers "F.Cu" "B.Cu") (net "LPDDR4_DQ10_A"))
 (segment (start 6.4 8.425) (end 6.8 8.75) (width 0.1) (layer "F.Cu") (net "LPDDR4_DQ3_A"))
 (via (at 6.8 8.75) (size 0.45) (drill 0.2) (layers "F.Cu" "B.Cu") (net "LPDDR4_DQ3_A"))
 (segment (start 8 8.425) (end 8.4 8.75) (width 0.1) (layer "F.Cu") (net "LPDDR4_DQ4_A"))
 (via (at 8.4 8.75) (size 0.45) (drill 0.2) (layers "F.Cu" "B.Cu") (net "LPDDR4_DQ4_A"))
 (segment (start 12 8.425) (end 11.6 8.75) (width 0.1) (layer "F.Cu") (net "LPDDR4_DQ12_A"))
 (via (at 11.6 8.75) (size 0.45) (drill 0.2) (layers "F.Cu" "B.Cu") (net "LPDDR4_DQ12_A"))
 (segment (start 13.6 8.425) (end 13.2 8.75) (width 0.1) (layer "F.Cu") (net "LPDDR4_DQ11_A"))
 (via (at 13.2 8.75) (size 0.45) (drill 0.2) (layers "F.Cu" "B.Cu") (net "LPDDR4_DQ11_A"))
 (segment (start 6.4 9.725) (end 6.8 10.05) (width 0.1) (layer "F.Cu") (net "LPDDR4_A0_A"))
 (via (at 6.8 10.05) (size 0.45) (drill 0.2) (layers "F.Cu" "B.Cu") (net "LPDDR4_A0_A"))
 (segment (start 8 9.725) (end 8.4 10.05) (width 0.1) (layer "F.Cu") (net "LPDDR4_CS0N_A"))
 (via (at 8.4 10.05) (size 0.45) (drill 0.2) (layers "F.Cu" "B.Cu") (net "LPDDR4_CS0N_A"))
 (segment (start 12 9.725) (end 11.6 10.05) (width 0.1) (layer "F.Cu") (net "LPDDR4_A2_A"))
 (via (at 11.6 10.05) (size 0.45) (drill 0.2) (layers "F.Cu" "B.Cu") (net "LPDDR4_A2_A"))
 (segment (start 12.8 9.725) (end 12.4 10.05) (width 0.1) (layer "F.Cu") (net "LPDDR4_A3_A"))
 (via (at 12.4 10.05) (size 0.45) (drill 0.2) (layers "F.Cu" "B.Cu") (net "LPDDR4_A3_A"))
 (segment (start 13.6 9.725) (end 13.2 10.05) (width 0.1) (layer "F.Cu") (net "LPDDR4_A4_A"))
 (via (at 13.2 10.05) (size 0.45) (drill 0.2) (layers "F.Cu" "B.Cu") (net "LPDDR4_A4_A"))
 (segment (start 6.4 10.375) (end 6.8 10.7) (width 0.1) (layer "F.Cu") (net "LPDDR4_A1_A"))
 (via (at 6.8 10.7) (size 0.45) (drill 0.2) (layers "F.Cu" "B.Cu") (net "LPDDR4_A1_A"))
 (segment (start 8 10.375) (end 8.4 10.7) (width 0.1) (layer "F.Cu") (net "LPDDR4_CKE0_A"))
 (via (at 8.4 10.7) (size 0.45) (drill 0.2) (layers "F.Cu" "B.Cu") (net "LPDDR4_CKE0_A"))
 (segment (start 11.2 10.375) (end 10.8 10.7) (width 0.1) (layer "F.Cu") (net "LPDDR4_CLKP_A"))
 (via (at 10.8 10.7) (size 0.45) (drill 0.2) (layers "F.Cu" "B.Cu") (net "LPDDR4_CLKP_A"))
 (segment (start 12 10.375) (end 11.6 10.7) (width 0.1) (layer "F.Cu") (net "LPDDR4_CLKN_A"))
 (via (at 11.6 10.7) (size 0.45) (drill 0.2) (layers "F.Cu" "B.Cu") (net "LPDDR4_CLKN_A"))
 (segment (start 13.6 10.375) (end 13.2 10.7) (width 0.1) (layer "F.Cu") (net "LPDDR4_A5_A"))
 (via (at 13.2 10.7) (size 0.45) (drill 0.2) (layers "F.Cu" "B.Cu") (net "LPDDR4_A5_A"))
 (segment (start 6.4 13.625) (end 6.8 13.3) (width 0.1) (layer "F.Cu") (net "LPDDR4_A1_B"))
 (via (at 6.8 13.3) (size 0.45) (drill 0.2) (layers "F.Cu" "B.Cu") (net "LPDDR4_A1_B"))
 (segment (start 8 13.625) (end 8.4 13.3) (width 0.1) (layer "F.Cu") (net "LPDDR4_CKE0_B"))
 (via (at 8.4 13.3) (size 0.45) (drill 0.2) (layers "F.Cu" "B.Cu") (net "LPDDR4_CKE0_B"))
 (segment (start 11.2 13.625) (end 10.8 13.3) (width 0.1) (layer "F.Cu") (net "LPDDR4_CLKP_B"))
 (via (at 10.8 13.3) (size 0.45) (drill 0.2) (layers "F.Cu" "B.Cu") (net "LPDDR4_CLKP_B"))
 (segment (start 12 13.625) (end 11.6 13.3) (width 0.1) (layer "F.Cu") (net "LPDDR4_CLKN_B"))
 (via (at 11.6 13.3) (size 0.45) (drill 0.2) (layers "F.Cu" "B.Cu") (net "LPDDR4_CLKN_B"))
 (segment (start 13.6 13.625) (end 13.2 13.3) (width 0.1) (layer "F.Cu") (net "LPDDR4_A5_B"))
 (via (at 13.2 13.3) (size 0.45) (drill 0.2) (layers "F.Cu" "B.Cu") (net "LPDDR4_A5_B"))
 (segment (start 6.4 14.275) (end 6.8 13.95) (width 0.1) (layer "F.Cu") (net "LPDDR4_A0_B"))
 (via (at 6.8 13.95) (size 0.45) (drill 0.2) (layers "F.Cu" "B.Cu") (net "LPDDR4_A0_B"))
 (segment (start 8 14.275) (end 8.4 13.95) (width 0.1) (layer "F.Cu") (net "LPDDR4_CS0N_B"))
 (via (at 8.4 13.95) (size 0.45) (drill 0.2) (layers "F.Cu" "B.Cu") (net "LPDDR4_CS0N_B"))
 (segment (start 12 14.275) (end 11.6 13.95) (width 0.1) (layer "F.Cu") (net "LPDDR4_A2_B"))
 (via (at 11.6 13.95) (size 0.45) (drill 0.2) (layers "F.Cu" "B.Cu") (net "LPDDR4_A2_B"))
 (segment (start 12.8 14.275) (end 12.4 13.95) (width 0.1) (layer "F.Cu") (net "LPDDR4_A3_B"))
 (via (at 12.4 13.95) (size 0.45) (drill 0.2) (layers "F.Cu" "B.Cu") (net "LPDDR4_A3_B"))
 (segment (start 13.6 14.275) (end 13.2 13.95) (width 0.1) (layer "F.Cu") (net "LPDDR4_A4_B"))
 (via (at 13.2 13.95) (size 0.45) (drill 0.2) (layers "F.Cu" "B.Cu") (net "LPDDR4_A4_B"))
 (segment (start 13.6 14.925) (end 13.2 14.6) (width 0.1) (layer "F.Cu") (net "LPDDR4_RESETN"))
 (via (at 13.2 14.6) (size 0.45) (drill 0.2) (layers "F.Cu" "B.Cu") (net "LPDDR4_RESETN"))
 (segment (start 6.4 15.575) (end 6.8 15.25) (width 0.1) (layer "F.Cu") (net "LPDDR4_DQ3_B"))
 (via (at 6.8 15.25) (size 0.45) (drill 0.2) (layers "F.Cu" "B.Cu") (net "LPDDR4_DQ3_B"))
 (segment (start 8 15.575) (end 8.4 15.25) (width 0.1) (layer "F.Cu") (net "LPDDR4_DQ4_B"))
 (via (at 8.4 15.25) (size 0.45) (drill 0.2) (layers "F.Cu" "B.Cu") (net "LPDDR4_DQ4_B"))
 (segment (start 12 15.575) (end 11.6 15.25) (width 0.1) (layer "F.Cu") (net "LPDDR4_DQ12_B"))
 (via (at 11.6 15.25) (size 0.45) (drill 0.2) (layers "F.Cu" "B.Cu") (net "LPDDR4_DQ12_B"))
 (segment (start 13.6 15.575) (end 13.2 15.25) (width 0.1) (layer "F.Cu") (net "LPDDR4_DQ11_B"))
 (via (at 13.2 15.25) (size 0.45) (drill 0.2) (layers "F.Cu" "B.Cu") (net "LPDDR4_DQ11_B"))
 (segment (start 6.4 16.225) (end 6.8 15.9) (width 0.1) (layer "F.Cu") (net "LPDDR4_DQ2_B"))
 (via (at 6.8 15.9) (size 0.45) (drill 0.2) (layers "F.Cu" "B.Cu") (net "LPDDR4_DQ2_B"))
 (segment (start 7.2 16.225) (end 7.6 15.9) (width 0.1) (layer "F.Cu") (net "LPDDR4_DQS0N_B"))
 (via (at 7.6 15.9) (size 0.45) (drill 0.2) (layers "F.Cu" "B.Cu") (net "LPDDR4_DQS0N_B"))
 (segment (start 8 16.225) (end 8.4 15.9) (width 0.1) (layer "F.Cu") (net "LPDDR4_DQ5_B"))
 (via (at 8.4 15.9) (size 0.45) (drill 0.2) (layers "F.Cu" "B.Cu") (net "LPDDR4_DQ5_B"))
 (segment (start 12 16.225) (end 11.6 15.9) (width 0.1) (layer "F.Cu") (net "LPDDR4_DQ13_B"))
 (via (at 11.6 15.9) (size 0.45) (drill 0.2) (layers "F.Cu" "B.Cu") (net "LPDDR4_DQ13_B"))
 (segment (start 12.8 16.225) (end 12.4 15.9) (width 0.1) (layer "F.Cu") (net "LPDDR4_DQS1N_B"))
 (via (at 12.4 15.9) (size 0.45) (drill 0.2) (layers "F.Cu" "B.Cu") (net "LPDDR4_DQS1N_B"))
 (segment (start 13.6 16.225) (end 13.2 15.9) (width 0.1) (layer "F.Cu") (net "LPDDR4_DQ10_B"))
 (via (at 13.2 15.9) (size 0.45) (drill 0.2) (layers "F.Cu" "B.Cu") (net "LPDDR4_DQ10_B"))
 (segment (start 7.2 16.875) (end 7.6 16.55) (width 0.1) (layer "F.Cu") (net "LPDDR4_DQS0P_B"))
 (via (at 7.6 16.55) (size 0.45) (drill 0.2) (layers "F.Cu" "B.Cu") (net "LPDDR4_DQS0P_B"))
 (segment (start 12.8 16.875) (end 12.4 16.55) (width 0.1) (layer "F.Cu") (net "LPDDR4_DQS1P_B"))
 (via (at 12.4 16.55) (size 0.45) (drill 0.2) (layers "F.Cu" "B.Cu") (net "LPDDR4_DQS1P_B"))
 (segment (start 6.4 17.525) (end 6.8 17.2) (width 0.1) (layer "F.Cu") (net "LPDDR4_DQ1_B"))
 (via (at 6.8 17.2) (size 0.45) (drill 0.2) (layers "F.Cu" "B.Cu") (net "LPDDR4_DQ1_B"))
 (segment (start 7.2 17.525) (end 7.6 17.2) (width 0.1) (layer "F.Cu") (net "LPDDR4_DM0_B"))
 (via (at 7.6 17.2) (size 0.45) (drill 0.2) (layers "F.Cu" "B.Cu") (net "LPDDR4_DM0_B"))
 (segment (start 8 17.525) (end 8.4 17.2) (width 0.1) (layer "F.Cu") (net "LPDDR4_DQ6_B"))
 (via (at 8.4 17.2) (size 0.45) (drill 0.2) (layers "F.Cu" "B.Cu") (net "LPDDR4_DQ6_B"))
 (segment (start 12 17.525) (end 11.6 17.2) (width 0.1) (layer "F.Cu") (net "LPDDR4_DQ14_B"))
 (via (at 11.6 17.2) (size 0.45) (drill 0.2) (layers "F.Cu" "B.Cu") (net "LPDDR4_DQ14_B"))
 (segment (start 12.8 17.525) (end 12.4 17.2) (width 0.1) (layer "F.Cu") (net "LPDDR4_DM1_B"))
 (via (at 12.4 17.2) (size 0.45) (drill 0.2) (layers "F.Cu" "B.Cu") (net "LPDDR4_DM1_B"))
 (segment (start 13.6 17.525) (end 13.2 17.2) (width 0.1) (layer "F.Cu") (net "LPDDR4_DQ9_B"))
 (via (at 13.2 17.2) (size 0.45) (drill 0.2) (layers "F.Cu" "B.Cu") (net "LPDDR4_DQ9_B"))
 (segment (start 6.4 18.175) (end 6.8 17.85) (width 0.1) (layer "F.Cu") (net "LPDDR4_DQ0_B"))
 (via (at 6.8 17.85) (size 0.45) (drill 0.2) (layers "F.Cu" "B.Cu") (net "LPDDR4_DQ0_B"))
 (segment (start 8 18.175) (end 8.4 17.85) (width 0.1) (layer "F.Cu") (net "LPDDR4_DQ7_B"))
 (via (at 8.4 17.85) (size 0.45) (drill 0.2) (layers "F.Cu" "B.Cu") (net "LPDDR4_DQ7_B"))
 (segment (start 12 18.175) (end 11.6 17.85) (width 0.1) (layer "F.Cu") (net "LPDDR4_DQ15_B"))
 (via (at 11.6 17.85) (size 0.45) (drill 0.2) (layers "F.Cu" "B.Cu") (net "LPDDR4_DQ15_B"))
 (segment (start 13.6 18.175) (end 13.2 17.85) (width 0.1) (layer "F.Cu") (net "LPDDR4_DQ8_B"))
 (via (at 13.2 17.85) (size 0.45) (drill 0.2) (layers "F.Cu" "B.Cu") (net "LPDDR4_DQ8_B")))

